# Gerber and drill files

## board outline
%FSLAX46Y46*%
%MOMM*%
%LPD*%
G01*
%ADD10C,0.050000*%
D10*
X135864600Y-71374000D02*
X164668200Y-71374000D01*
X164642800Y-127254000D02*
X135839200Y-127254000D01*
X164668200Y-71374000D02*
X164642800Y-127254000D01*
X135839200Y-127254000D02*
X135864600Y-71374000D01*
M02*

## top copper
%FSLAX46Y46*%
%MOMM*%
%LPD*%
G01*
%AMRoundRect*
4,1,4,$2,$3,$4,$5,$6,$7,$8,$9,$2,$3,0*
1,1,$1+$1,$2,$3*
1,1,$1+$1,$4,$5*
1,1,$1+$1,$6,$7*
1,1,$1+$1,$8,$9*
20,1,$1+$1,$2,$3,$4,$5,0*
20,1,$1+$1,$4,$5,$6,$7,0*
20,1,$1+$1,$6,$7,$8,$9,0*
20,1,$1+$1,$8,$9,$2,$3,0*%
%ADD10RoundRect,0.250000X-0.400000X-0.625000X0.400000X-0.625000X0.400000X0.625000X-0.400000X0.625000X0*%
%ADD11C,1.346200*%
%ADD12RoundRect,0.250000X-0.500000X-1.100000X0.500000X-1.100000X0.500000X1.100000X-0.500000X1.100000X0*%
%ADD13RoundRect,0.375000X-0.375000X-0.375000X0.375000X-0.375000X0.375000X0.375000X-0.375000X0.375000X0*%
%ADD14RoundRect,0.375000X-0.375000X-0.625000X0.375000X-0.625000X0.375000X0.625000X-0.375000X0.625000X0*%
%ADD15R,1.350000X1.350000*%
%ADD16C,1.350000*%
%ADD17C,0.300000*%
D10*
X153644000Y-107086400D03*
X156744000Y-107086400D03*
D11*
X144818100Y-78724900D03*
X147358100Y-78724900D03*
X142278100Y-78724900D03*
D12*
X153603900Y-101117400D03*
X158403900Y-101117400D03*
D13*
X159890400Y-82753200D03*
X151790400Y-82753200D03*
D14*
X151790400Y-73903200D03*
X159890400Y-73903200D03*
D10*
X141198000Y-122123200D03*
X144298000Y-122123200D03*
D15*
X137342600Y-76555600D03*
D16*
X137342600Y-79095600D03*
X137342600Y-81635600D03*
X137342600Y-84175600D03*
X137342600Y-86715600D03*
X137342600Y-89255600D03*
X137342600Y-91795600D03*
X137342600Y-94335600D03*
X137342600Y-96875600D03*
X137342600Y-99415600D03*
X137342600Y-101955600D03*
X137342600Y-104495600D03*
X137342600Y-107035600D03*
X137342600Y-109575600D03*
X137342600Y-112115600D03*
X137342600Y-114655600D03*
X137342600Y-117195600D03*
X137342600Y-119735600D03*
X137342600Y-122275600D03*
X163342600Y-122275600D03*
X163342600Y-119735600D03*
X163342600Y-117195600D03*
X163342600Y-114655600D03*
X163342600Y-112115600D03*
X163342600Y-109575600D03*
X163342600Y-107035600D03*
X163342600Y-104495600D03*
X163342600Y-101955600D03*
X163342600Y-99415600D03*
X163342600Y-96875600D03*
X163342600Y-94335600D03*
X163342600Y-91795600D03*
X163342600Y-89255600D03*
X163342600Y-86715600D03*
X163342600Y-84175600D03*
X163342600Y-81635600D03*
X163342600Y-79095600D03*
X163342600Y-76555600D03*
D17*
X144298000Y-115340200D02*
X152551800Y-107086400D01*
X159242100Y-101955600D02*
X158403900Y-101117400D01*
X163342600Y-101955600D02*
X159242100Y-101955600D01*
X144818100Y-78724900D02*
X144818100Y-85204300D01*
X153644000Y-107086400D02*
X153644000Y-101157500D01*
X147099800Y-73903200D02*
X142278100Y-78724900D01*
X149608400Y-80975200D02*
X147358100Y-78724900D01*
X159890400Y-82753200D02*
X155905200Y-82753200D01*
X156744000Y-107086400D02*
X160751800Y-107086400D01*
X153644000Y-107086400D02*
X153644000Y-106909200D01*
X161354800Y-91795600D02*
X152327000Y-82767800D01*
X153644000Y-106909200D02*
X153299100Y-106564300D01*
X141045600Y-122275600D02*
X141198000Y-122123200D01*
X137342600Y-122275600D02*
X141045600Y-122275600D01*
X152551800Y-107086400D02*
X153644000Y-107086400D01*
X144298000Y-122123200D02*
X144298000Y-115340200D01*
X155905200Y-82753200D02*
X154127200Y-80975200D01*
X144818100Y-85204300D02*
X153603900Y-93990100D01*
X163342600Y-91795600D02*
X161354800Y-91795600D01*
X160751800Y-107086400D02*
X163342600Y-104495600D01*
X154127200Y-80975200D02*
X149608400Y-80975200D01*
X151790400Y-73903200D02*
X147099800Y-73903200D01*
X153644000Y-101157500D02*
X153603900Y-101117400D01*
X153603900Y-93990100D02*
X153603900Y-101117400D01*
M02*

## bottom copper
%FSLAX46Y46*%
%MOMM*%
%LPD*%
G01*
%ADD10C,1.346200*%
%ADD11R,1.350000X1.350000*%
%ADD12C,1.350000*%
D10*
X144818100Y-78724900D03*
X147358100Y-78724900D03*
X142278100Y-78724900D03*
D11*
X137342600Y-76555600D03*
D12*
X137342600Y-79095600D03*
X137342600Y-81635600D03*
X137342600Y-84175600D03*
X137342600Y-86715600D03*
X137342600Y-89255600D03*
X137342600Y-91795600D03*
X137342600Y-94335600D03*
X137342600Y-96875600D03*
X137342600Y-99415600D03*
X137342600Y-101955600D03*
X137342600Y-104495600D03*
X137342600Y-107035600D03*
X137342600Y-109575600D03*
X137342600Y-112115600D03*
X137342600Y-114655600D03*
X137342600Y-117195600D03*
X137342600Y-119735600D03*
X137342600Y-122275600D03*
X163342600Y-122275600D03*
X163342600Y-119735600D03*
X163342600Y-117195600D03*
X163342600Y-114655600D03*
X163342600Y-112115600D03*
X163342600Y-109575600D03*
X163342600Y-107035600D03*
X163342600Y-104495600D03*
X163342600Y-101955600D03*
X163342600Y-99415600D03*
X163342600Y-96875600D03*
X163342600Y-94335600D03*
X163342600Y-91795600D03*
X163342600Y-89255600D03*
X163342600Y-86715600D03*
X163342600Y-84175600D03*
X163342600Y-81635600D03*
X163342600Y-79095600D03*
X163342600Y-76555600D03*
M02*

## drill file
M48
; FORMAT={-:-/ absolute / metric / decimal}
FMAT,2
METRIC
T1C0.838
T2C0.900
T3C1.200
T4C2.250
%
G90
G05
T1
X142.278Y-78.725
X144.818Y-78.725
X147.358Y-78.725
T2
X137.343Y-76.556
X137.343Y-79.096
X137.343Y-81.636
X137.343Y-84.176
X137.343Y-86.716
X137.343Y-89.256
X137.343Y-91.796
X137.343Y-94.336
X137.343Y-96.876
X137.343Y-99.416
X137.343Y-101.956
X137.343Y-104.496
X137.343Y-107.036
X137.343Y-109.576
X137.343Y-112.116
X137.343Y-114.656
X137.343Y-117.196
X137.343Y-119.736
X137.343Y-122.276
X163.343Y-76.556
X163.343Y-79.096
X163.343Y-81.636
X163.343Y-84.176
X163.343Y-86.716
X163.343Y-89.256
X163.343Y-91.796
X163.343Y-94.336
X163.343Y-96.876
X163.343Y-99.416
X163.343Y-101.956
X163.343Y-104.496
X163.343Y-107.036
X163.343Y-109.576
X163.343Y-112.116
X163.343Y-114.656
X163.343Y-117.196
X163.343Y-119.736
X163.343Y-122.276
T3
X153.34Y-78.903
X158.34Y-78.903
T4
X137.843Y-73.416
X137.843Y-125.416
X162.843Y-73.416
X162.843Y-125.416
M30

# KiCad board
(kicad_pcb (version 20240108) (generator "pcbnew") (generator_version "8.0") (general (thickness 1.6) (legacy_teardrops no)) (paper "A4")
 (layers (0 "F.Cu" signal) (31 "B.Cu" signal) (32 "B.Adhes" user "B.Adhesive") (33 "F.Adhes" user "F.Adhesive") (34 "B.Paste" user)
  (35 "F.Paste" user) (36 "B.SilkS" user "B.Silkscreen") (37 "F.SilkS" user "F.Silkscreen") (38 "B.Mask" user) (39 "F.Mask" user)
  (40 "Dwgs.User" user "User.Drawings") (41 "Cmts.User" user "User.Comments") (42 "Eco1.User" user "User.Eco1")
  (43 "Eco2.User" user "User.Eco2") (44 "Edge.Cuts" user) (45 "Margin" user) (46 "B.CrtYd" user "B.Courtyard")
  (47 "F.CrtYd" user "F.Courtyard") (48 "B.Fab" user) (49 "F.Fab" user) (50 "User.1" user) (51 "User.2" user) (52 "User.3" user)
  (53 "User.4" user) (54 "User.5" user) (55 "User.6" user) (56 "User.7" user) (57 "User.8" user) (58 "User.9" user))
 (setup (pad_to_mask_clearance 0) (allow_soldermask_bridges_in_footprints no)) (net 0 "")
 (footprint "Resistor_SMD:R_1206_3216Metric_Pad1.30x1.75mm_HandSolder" (layer "F.Cu") (at 155.194 107.0864)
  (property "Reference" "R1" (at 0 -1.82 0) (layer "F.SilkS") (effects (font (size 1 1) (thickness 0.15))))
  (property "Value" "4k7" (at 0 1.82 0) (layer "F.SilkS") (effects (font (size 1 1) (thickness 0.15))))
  (pad "1" smd roundrect (at -1.55 0) (size 1.3 1.75) (layers "F.Cu" "F.Paste" "F.Mask") (roundrect_rratio 0.192308))
  (pad "2" smd roundrect (at 1.55 0) (size 1.3 1.75) (layers "F.Cu" "F.Paste" "F.Mask") (roundrect_rratio 0.192308)))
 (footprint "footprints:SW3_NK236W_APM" (layer "F.Cu") (at 144.8181 78.7249 180)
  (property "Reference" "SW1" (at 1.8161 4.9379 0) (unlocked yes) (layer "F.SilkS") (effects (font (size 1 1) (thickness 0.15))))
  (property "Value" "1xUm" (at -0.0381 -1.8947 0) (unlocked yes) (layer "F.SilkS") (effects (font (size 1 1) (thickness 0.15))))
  (pad "1" thru_hole circle (at 0 0 180) (size 1.3462 1.3462) (drill 0.8382) (layers "*.Cu" "*.Mask") (remove_unused_layers no))
  (pad "2" thru_hole circle (at -2.54 0 180) (size 1.3462 1.3462) (drill 0.8382) (layers "*.Cu" "*.Mask") (remove_unused_layers no))
  (pad "3" thru_hole circle (at 2.54 0 180) (size 1.3462 1.3462) (drill 0.8382) (layers "*.Cu" "*.Mask") (remove_unused_layers no)))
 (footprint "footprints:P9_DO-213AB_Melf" (layer "F.Cu") (at 153.6039 101.1174)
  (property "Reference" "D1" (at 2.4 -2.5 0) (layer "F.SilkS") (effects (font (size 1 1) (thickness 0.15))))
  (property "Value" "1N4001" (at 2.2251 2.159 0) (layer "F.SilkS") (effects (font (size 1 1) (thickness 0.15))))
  (pad "1" smd roundrect (at 0 0) (size 1.5 2.7) (layers "F.Cu" "F.Paste" "F.Mask") (roundrect_rratio 0.1666666667))
  (pad "2" smd roundrect (at 4.8 0) (size 1.5 2.7) (layers "F.Cu" "F.Paste" "F.Mask") (roundrect_rratio 0.1666666667)))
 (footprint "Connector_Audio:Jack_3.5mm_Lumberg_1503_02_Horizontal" (layer "F.Cu") (at 155.8404 76.4032)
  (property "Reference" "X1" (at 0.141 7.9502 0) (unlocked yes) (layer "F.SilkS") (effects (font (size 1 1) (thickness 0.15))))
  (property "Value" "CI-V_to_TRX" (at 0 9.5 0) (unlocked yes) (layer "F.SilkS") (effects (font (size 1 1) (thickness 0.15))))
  (pad "" np_thru_hole circle (at -2.5 2.5) (size 1.2 1.2) (drill 1.2) (layers "F&B.Cu" "*.Mask"))
  (pad "" np_thru_hole circle (at 2.5 2.5) (size 1.2 1.2) (drill 1.2) (layers "F&B.Cu" "*.Mask"))
  (pad "R" smd roundrect (at 4.05 6.35) (size 1.5 1.5) (layers "F.Cu" "F.Paste" "F.Mask") (roundrect_rratio 0.25))
  (pad "S" smd roundrect (at -4.05 6.35) (size 1.5 1.5) (layers "F.Cu" "F.Paste" "F.Mask") (roundrect_rratio 0.25))
  (pad "T" smd roundrect (at -4.05 -2.5) (size 1.5 2) (layers "F.Cu" "F.Paste" "F.Mask") (roundrect_rratio 0.25))
  (pad "T" smd roundrect (at 4.05 -2.5) (size 1.5 2) (layers "F.Cu" "F.Paste" "F.Mask") (roundrect_rratio 0.25)))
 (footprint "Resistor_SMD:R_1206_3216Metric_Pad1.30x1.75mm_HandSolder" (layer "F.Cu") (at 142.748 122.1232)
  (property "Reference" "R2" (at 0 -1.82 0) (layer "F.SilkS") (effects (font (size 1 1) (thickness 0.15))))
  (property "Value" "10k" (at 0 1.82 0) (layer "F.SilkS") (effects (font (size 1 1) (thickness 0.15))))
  (pad "1" smd roundrect (at -1.55 0) (size 1.3 1.75) (layers "F.Cu" "F.Paste" "F.Mask") (roundrect_rratio 0.192308))
  (pad "2" smd roundrect (at 1.55 0) (size 1.3 1.75) (layers "F.Cu" "F.Paste" "F.Mask") (roundrect_rratio 0.192308)))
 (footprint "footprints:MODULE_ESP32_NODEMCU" (layer "B.Cu") (at 150.3426 99.4156 180)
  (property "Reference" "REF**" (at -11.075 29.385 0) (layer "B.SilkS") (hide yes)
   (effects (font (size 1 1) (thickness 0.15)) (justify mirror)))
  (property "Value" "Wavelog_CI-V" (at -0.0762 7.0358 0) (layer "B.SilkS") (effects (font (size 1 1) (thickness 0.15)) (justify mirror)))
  (pad "" np_thru_hole circle (at -12.5 -26 180) (size 2.25 2.25) (drill 2.25) (layers "*.Cu" "*.Mask"))
  (pad "" np_thru_hole circle (at -12.5 26 180) (size 2.25 2.25) (drill 2.25) (layers "*.Cu" "*.Mask"))
  (pad "" np_thru_hole circle (at 12.5 -26 180) (size 2.25 2.25) (drill 2.25) (layers "*.Cu" "*.Mask"))
  (pad "" np_thru_hole circle (at 12.5 26 180) (size 2.25 2.25) (drill 2.25) (layers "*.Cu" "*.Mask"))
  (pad "J4_1" thru_hole rect (at 13 22.86 180) (size 1.35 1.35) (drill 0.9) (layers "*.Cu" "*.Mask") (remove_unused_layers no)
   (solder_mask_margin 0.102))
  (pad "J4_2" thru_hole circle (at 13 20.32 180) (size 1.35 1.35) (drill 0.9) (layers "*.Cu" "*.Mask") (remove_unused_layers no)
   (solder_mask_margin 0.102))
  (pad "J4_3" thru_hole circle (at 13 17.78 180) (size 1.35 1.35) (drill 0.9) (layers "*.Cu" "*.Mask") (remove_unused_layers no)
   (solder_mask_margin 0.102))
  (pad "J4_4" thru_hole circle (at 13 15.24 180) (size 1.35 1.35) (drill 0.9) (layers "*.Cu" "*.Mask") (remove_unused_layers no)
   (solder_mask_margin 0.102))
  (pad "J4_5" thru_hole circle (at 13 12.7 180) (size 1.35 1.35) (drill 0.9) (layers "*.Cu" "*.Mask") (remove_unused_layers no)
   (solder_mask_margin 0.102))
  (pad "J4_6" thru_hole circle (at 13 10.16 180) (size 1.35 1.35) (drill 0.9) (layers "*.Cu" "*.Mask") (remove_unused_layers no)
   (solder_mask_margin 0.102))
  (pad "J4_7" thru_hole circle (at 13 7.62 180) (size 1.35 1.35) (drill 0.9) (layers "*.Cu" "*.Mask") (remove_unused_layers no)
   (solder_mask_margin 0.102))
  (pad "J4_8" thru_hole circle (at 13 5.08 180) (size 1.35 1.35) (drill 0.9) (layers "*.Cu" "*.Mask") (remove_unused_layers no)
   (solder_mask_margin 0.102))
  (pad "J4_9" thru_hole circle (at 13 2.54 180) (size 1.35 1.35) (drill 0.9) (layers "*.Cu" "*.Mask") (remove_unused_layers no)
   (solder_mask_margin 0.102))
  (pad "J4_10" thru_hole circle (at 13 0 180) (size 1.35 1.35) (drill 0.9) (layers "*.Cu" "*.Mask") (remove_unused_layers no)
   (solder_mask_margin 0.102))
  (pad "J4_11" thru_hole circle (at 13 -2.54 180) (size 1.35 1.35) (drill 0.9) (layers "*.Cu" "*.Mask") (remove_unused_layers no)
   (solder_mask_margin 0.102))
  (pad "J4_12" thru_hole circle (at 13 -5.08 180) (size 1.35 1.35) (drill 0.9) (layers "*.Cu" "*.Mask") (remove_unused_layers no)
   (solder_mask_margin 0.102))
  (pad "J4_13" thru_hole circle (at 13 -7.62 180) (size 1.35 1.35) (drill 0.9) (layers "*.Cu" "*.Mask") (remove_unused_layers no)
   (solder_mask_margin 0.102))
  (pad "J4_14" thru_hole circle (at 13 -10.16 180) (size 1.35 1.35) (drill 0.9) (layers "*.Cu" "*.Mask") (remove_unused_layers no)
   (solder_mask_margin 0.102))
  (pad "J4_15" thru_hole circle (at 13 -12.7 180) (size 1.35 1.35) (drill 0.9) (layers "*.Cu" "*.Mask") (remove_unused_layers no)
   (solder_mask_margin 0.102))
  (pad "J4_16" thru_hole circle (at 13 -15.24 180) (size 1.35 1.35) (drill 0.9) (layers "*.Cu" "*.Mask") (remove_unused_layers no)
   (solder_mask_margin 0.102))
  (pad "J4_17" thru_hole circle (at 13 -17.78 180) (size 1.35 1.35) (drill 0.9) (layers "*.Cu" "*.Mask") (remove_unused_layers no)
   (solder_mask_margin 0.102))
  (pad "J4_18" thru_hole circle (at 13 -20.32 180) (size 1.35 1.35) (drill 0.9) (layers "*.Cu" "*.Mask") (remove_unused_layers no)
   (solder_mask_margin 0.102))
  (pad "J4_19" thru_hole circle (at 13 -22.86 180) (size 1.35 1.35) (drill 0.9) (layers "*.Cu" "*.Mask") (remove_unused_layers no)
   (solder_mask_margin 0.102))
  (pad "J5_1" thru_hole circle (at -13 -22.86 180) (size 1.35 1.35) (drill 0.9) (layers "*.Cu" "*.Mask") (remove_unused_layers no)
   (solder_mask_margin 0.102))
  (pad "J5_2" thru_hole circle (at -13 -20.32 180) (size 1.35 1.35) (drill 0.9) (layers "*.Cu" "*.Mask") (remove_unused_layers no)
   (solder_mask_margin 0.102))
  (pad "J5_3" thru_hole circle (at -13 -17.78 180) (size 1.35 1.35) (drill 0.9) (layers "*.Cu" "*.Mask") (remove_unused_layers no)
   (solder_mask_margin 0.102))
  (pad "J5_4" thru_hole circle (at -13 -15.24 180) (size 1.35 1.35) (drill 0.9) (layers "*.Cu" "*.Mask") (remove_unused_layers no)
   (solder_mask_margin 0.102))
  (pad "J5_5" thru_hole circle (at -13 -12.7 180) (size 1.35 1.35) (drill 0.9) (layers "*.Cu" "*.Mask") (remove_unused_layers no)
   (solder_mask_margin 0.102))
  (pad "J5_6" thru_hole circle (at -13 -10.16 180) (size 1.35 1.35) (drill 0.9) (layers "*.Cu" "*.Mask") (remove_unused_layers no)
   (solder_mask_margin 0.102))
  (pad "J5_7" thru_hole circle (at -13 -7.62 180) (size 1.35 1.35) (drill 0.9) (layers "*.Cu" "*.Mask") (remove_unused_layers no)
   (solder_mask_margin 0.102))
  (pad "J5_8" thru_hole circle (at -13 -5.08 180) (size 1.35 1.35) (drill 0.9) (layers "*.Cu" "*.Mask") (remove_unused_layers no)
   (solder_mask_margin 0.102))
  (pad "J5_9" thru_hole circle (at -13 -2.54 180) (size 1.35 1.35) (drill 0.9) (layers "*.Cu" "*.Mask") (remove_unused_layers no)
   (solder_mask_margin 0.102))
  (pad "J5_10" thru_hole circle (at -13 0 180) (size 1.35 1.35) (drill 0.9) (layers "*.Cu" "*.Mask") (remove_unused_layers no)
   (solder_mask_margin 0.102))
  (pad "J5_11" thru_hole circle (at -13 2.54 180) (size 1.35 1.35) (drill 0.9) (layers "*.Cu" "*.Mask") (remove_unused_layers no)
   (solder_mask_margin 0.102))
  (pad "J5_12" thru_hole circle (at -13 5.08 180) (size 1.35 1.35) (drill 0.9) (layers "*.Cu" "*.Mask") (remove_unused_layers no)
   (solder_mask_margin 0.102))
  (pad "J5_13" thru_hole circle (at -13 7.62 180) (size 1.35 1.35) (drill 0.9) (layers "*.Cu" "*.Mask") (remove_unused_layers no)
   (solder_mask_margin 0.102))
  (pad "J5_14" thru_hole circle (at -13 10.16 180) (size 1.35 1.35) (drill 0.9) (layers "*.Cu" "*.Mask") (remove_unused_layers no)
   (solder_mask_margin 0.102))
  (pad "J5_15" thru_hole circle (at -13 12.7 180) (size 1.35 1.35) (drill 0.9) (layers "*.Cu" "*.Mask") (remove_unused_layers no)
   (solder_mask_margin 0.102))
  (pad "J5_16" thru_hole circle (at -13 15.24 180) (size 1.35 1.35) (drill 0.9) (layers "*.Cu" "*.Mask") (remove_unused_layers no)
   (solder_mask_margin 0.102))
  (pad "J5_17" thru_hole circle (at -13 17.78 180) (size 1.35 1.35) (drill 0.9) (layers "*.Cu" "*.Mask") (remove_unused_layers no)
   (solder_mask_margin 0.102))
  (pad "J5_18" thru_hole circle (at -13 20.32 180) (size 1.35 1.35) (drill 0.9) (layers "*.Cu" "*.Mask") (remove_unused_layers no)
   (solder_mask_margin 0.102))
  (pad "J5_19" thru_hole circle (at -13 22.86 180) (size 1.35 1.35) (drill 0.9) (layers "*.Cu" "*.Mask") (remove_unused_layers no)
   (solder_mask_margin 0.102)))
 (gr_line (start 135.8646 71.374) (end 164.6682 71.374) (stroke (width 0.05) (type default)) (layer "Edge.Cuts"))
 (gr_line (start 164.6428 127.254) (end 135.8392 127.254) (stroke (width 0.05) (type default)) (layer "Edge.Cuts"))
 (gr_line (start 164.6682 71.374) (end 164.6428 127.254) (stroke (width 0.05) (type default)) (layer "Edge.Cuts"))
 (gr_line (start 135.8392 127.254) (end 135.8646 71.374) (stroke (width 0.05) (type default)) (layer "Edge.Cuts"))
 (segment (start 144.298 115.3402) (end 152.5518 107.0864) (width 0.3) (layer "F.Cu") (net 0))
 (segment (start 159.2421 101.9556) (end 158.4039 101.1174) (width 0.3) (layer "F.Cu") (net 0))
 (segment (start 163.3426 101.9556) (end 159.2421 101.9556) (width 0.3) (layer "F.Cu") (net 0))
 (segment (start 144.8181 78.7249) (end 144.8181 85.2043) (width 0.3) (layer "F.Cu") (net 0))
 (segment (start 153.644 107.0864) (end 153.644 101.1575) (width 0.3) (layer "F.Cu") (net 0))
 (segment (start 147.0998 73.9032) (end 142.2781 78.7249) (width 0.3) (layer "F.Cu") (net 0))
 (segment (start 149.6084 80.9752) (end 147.3581 78.7249) (width 0.3) (layer "F.Cu") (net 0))
 (segment (start 159.8904 82.7532) (end 155.9052 82.7532) (width 0.3) (layer "F.Cu") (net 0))
 (segment (start 156.744 107.0864) (end 160.7518 107.0864) (width 0.3) (layer "F.Cu") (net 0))
 (segment (start 153.644 107.0864) (end 153.644 106.9092) (width 0.3) (layer "F.Cu") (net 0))
 (segment (start 161.3548 91.7956) (end 152.327 82.7678) (width 0.3) (layer "F.Cu") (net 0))
 (segment (start 153.644 106.9092) (end 153.2991 106.5643) (width 0.3) (layer "F.Cu") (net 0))
 (segment (start 141.0456 122.2756) (end 141.198 122.1232) (width 0.3) (layer "F.Cu") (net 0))
 (segment (start 137.3426 122.2756) (end 141.0456 122.2756) (width 0.3) (layer "F.Cu") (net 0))
 (segment (start 152.5518 107.0864) (end 153.644 107.0864) (width 0.3) (layer "F.Cu") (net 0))
 (segment (start 144.298 122.1232) (end 144.298 115.3402) (width 0.3) (layer "F.Cu") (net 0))
 (segment (start 155.9052 82.7532) (end 154.1272 80.9752) (width 0.3) (layer "F.Cu") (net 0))
 (segment (start 144.8181 85.2043) (end 153.6039 93.9901) (width 0.3) (layer "F.Cu") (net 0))
 (segment (start 163.3426 91.7956) (end 161.3548 91.7956) (width 0.3) (layer "F.Cu") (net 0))
 (segment (start 160.7518 107.0864) (end 163.3426 104.4956) (width 0.3) (layer "F.Cu") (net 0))
 (segment (start 154.1272 80.9752) (end 149.6084 80.9752) (width 0.3) (layer "F.Cu") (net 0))
 (segment (start 151.7904 73.9032) (end 147.0998 73.9032) (width 0.3) (layer "F.Cu") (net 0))
 (segment (start 153.644 101.1575) (end 153.6039 101.1174) (width 0.3) (layer "F.Cu") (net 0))
 (segment (start 153.6039 93.9901) (end 153.6039 101.1174) (width 0.3) (layer "F.Cu") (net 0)))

